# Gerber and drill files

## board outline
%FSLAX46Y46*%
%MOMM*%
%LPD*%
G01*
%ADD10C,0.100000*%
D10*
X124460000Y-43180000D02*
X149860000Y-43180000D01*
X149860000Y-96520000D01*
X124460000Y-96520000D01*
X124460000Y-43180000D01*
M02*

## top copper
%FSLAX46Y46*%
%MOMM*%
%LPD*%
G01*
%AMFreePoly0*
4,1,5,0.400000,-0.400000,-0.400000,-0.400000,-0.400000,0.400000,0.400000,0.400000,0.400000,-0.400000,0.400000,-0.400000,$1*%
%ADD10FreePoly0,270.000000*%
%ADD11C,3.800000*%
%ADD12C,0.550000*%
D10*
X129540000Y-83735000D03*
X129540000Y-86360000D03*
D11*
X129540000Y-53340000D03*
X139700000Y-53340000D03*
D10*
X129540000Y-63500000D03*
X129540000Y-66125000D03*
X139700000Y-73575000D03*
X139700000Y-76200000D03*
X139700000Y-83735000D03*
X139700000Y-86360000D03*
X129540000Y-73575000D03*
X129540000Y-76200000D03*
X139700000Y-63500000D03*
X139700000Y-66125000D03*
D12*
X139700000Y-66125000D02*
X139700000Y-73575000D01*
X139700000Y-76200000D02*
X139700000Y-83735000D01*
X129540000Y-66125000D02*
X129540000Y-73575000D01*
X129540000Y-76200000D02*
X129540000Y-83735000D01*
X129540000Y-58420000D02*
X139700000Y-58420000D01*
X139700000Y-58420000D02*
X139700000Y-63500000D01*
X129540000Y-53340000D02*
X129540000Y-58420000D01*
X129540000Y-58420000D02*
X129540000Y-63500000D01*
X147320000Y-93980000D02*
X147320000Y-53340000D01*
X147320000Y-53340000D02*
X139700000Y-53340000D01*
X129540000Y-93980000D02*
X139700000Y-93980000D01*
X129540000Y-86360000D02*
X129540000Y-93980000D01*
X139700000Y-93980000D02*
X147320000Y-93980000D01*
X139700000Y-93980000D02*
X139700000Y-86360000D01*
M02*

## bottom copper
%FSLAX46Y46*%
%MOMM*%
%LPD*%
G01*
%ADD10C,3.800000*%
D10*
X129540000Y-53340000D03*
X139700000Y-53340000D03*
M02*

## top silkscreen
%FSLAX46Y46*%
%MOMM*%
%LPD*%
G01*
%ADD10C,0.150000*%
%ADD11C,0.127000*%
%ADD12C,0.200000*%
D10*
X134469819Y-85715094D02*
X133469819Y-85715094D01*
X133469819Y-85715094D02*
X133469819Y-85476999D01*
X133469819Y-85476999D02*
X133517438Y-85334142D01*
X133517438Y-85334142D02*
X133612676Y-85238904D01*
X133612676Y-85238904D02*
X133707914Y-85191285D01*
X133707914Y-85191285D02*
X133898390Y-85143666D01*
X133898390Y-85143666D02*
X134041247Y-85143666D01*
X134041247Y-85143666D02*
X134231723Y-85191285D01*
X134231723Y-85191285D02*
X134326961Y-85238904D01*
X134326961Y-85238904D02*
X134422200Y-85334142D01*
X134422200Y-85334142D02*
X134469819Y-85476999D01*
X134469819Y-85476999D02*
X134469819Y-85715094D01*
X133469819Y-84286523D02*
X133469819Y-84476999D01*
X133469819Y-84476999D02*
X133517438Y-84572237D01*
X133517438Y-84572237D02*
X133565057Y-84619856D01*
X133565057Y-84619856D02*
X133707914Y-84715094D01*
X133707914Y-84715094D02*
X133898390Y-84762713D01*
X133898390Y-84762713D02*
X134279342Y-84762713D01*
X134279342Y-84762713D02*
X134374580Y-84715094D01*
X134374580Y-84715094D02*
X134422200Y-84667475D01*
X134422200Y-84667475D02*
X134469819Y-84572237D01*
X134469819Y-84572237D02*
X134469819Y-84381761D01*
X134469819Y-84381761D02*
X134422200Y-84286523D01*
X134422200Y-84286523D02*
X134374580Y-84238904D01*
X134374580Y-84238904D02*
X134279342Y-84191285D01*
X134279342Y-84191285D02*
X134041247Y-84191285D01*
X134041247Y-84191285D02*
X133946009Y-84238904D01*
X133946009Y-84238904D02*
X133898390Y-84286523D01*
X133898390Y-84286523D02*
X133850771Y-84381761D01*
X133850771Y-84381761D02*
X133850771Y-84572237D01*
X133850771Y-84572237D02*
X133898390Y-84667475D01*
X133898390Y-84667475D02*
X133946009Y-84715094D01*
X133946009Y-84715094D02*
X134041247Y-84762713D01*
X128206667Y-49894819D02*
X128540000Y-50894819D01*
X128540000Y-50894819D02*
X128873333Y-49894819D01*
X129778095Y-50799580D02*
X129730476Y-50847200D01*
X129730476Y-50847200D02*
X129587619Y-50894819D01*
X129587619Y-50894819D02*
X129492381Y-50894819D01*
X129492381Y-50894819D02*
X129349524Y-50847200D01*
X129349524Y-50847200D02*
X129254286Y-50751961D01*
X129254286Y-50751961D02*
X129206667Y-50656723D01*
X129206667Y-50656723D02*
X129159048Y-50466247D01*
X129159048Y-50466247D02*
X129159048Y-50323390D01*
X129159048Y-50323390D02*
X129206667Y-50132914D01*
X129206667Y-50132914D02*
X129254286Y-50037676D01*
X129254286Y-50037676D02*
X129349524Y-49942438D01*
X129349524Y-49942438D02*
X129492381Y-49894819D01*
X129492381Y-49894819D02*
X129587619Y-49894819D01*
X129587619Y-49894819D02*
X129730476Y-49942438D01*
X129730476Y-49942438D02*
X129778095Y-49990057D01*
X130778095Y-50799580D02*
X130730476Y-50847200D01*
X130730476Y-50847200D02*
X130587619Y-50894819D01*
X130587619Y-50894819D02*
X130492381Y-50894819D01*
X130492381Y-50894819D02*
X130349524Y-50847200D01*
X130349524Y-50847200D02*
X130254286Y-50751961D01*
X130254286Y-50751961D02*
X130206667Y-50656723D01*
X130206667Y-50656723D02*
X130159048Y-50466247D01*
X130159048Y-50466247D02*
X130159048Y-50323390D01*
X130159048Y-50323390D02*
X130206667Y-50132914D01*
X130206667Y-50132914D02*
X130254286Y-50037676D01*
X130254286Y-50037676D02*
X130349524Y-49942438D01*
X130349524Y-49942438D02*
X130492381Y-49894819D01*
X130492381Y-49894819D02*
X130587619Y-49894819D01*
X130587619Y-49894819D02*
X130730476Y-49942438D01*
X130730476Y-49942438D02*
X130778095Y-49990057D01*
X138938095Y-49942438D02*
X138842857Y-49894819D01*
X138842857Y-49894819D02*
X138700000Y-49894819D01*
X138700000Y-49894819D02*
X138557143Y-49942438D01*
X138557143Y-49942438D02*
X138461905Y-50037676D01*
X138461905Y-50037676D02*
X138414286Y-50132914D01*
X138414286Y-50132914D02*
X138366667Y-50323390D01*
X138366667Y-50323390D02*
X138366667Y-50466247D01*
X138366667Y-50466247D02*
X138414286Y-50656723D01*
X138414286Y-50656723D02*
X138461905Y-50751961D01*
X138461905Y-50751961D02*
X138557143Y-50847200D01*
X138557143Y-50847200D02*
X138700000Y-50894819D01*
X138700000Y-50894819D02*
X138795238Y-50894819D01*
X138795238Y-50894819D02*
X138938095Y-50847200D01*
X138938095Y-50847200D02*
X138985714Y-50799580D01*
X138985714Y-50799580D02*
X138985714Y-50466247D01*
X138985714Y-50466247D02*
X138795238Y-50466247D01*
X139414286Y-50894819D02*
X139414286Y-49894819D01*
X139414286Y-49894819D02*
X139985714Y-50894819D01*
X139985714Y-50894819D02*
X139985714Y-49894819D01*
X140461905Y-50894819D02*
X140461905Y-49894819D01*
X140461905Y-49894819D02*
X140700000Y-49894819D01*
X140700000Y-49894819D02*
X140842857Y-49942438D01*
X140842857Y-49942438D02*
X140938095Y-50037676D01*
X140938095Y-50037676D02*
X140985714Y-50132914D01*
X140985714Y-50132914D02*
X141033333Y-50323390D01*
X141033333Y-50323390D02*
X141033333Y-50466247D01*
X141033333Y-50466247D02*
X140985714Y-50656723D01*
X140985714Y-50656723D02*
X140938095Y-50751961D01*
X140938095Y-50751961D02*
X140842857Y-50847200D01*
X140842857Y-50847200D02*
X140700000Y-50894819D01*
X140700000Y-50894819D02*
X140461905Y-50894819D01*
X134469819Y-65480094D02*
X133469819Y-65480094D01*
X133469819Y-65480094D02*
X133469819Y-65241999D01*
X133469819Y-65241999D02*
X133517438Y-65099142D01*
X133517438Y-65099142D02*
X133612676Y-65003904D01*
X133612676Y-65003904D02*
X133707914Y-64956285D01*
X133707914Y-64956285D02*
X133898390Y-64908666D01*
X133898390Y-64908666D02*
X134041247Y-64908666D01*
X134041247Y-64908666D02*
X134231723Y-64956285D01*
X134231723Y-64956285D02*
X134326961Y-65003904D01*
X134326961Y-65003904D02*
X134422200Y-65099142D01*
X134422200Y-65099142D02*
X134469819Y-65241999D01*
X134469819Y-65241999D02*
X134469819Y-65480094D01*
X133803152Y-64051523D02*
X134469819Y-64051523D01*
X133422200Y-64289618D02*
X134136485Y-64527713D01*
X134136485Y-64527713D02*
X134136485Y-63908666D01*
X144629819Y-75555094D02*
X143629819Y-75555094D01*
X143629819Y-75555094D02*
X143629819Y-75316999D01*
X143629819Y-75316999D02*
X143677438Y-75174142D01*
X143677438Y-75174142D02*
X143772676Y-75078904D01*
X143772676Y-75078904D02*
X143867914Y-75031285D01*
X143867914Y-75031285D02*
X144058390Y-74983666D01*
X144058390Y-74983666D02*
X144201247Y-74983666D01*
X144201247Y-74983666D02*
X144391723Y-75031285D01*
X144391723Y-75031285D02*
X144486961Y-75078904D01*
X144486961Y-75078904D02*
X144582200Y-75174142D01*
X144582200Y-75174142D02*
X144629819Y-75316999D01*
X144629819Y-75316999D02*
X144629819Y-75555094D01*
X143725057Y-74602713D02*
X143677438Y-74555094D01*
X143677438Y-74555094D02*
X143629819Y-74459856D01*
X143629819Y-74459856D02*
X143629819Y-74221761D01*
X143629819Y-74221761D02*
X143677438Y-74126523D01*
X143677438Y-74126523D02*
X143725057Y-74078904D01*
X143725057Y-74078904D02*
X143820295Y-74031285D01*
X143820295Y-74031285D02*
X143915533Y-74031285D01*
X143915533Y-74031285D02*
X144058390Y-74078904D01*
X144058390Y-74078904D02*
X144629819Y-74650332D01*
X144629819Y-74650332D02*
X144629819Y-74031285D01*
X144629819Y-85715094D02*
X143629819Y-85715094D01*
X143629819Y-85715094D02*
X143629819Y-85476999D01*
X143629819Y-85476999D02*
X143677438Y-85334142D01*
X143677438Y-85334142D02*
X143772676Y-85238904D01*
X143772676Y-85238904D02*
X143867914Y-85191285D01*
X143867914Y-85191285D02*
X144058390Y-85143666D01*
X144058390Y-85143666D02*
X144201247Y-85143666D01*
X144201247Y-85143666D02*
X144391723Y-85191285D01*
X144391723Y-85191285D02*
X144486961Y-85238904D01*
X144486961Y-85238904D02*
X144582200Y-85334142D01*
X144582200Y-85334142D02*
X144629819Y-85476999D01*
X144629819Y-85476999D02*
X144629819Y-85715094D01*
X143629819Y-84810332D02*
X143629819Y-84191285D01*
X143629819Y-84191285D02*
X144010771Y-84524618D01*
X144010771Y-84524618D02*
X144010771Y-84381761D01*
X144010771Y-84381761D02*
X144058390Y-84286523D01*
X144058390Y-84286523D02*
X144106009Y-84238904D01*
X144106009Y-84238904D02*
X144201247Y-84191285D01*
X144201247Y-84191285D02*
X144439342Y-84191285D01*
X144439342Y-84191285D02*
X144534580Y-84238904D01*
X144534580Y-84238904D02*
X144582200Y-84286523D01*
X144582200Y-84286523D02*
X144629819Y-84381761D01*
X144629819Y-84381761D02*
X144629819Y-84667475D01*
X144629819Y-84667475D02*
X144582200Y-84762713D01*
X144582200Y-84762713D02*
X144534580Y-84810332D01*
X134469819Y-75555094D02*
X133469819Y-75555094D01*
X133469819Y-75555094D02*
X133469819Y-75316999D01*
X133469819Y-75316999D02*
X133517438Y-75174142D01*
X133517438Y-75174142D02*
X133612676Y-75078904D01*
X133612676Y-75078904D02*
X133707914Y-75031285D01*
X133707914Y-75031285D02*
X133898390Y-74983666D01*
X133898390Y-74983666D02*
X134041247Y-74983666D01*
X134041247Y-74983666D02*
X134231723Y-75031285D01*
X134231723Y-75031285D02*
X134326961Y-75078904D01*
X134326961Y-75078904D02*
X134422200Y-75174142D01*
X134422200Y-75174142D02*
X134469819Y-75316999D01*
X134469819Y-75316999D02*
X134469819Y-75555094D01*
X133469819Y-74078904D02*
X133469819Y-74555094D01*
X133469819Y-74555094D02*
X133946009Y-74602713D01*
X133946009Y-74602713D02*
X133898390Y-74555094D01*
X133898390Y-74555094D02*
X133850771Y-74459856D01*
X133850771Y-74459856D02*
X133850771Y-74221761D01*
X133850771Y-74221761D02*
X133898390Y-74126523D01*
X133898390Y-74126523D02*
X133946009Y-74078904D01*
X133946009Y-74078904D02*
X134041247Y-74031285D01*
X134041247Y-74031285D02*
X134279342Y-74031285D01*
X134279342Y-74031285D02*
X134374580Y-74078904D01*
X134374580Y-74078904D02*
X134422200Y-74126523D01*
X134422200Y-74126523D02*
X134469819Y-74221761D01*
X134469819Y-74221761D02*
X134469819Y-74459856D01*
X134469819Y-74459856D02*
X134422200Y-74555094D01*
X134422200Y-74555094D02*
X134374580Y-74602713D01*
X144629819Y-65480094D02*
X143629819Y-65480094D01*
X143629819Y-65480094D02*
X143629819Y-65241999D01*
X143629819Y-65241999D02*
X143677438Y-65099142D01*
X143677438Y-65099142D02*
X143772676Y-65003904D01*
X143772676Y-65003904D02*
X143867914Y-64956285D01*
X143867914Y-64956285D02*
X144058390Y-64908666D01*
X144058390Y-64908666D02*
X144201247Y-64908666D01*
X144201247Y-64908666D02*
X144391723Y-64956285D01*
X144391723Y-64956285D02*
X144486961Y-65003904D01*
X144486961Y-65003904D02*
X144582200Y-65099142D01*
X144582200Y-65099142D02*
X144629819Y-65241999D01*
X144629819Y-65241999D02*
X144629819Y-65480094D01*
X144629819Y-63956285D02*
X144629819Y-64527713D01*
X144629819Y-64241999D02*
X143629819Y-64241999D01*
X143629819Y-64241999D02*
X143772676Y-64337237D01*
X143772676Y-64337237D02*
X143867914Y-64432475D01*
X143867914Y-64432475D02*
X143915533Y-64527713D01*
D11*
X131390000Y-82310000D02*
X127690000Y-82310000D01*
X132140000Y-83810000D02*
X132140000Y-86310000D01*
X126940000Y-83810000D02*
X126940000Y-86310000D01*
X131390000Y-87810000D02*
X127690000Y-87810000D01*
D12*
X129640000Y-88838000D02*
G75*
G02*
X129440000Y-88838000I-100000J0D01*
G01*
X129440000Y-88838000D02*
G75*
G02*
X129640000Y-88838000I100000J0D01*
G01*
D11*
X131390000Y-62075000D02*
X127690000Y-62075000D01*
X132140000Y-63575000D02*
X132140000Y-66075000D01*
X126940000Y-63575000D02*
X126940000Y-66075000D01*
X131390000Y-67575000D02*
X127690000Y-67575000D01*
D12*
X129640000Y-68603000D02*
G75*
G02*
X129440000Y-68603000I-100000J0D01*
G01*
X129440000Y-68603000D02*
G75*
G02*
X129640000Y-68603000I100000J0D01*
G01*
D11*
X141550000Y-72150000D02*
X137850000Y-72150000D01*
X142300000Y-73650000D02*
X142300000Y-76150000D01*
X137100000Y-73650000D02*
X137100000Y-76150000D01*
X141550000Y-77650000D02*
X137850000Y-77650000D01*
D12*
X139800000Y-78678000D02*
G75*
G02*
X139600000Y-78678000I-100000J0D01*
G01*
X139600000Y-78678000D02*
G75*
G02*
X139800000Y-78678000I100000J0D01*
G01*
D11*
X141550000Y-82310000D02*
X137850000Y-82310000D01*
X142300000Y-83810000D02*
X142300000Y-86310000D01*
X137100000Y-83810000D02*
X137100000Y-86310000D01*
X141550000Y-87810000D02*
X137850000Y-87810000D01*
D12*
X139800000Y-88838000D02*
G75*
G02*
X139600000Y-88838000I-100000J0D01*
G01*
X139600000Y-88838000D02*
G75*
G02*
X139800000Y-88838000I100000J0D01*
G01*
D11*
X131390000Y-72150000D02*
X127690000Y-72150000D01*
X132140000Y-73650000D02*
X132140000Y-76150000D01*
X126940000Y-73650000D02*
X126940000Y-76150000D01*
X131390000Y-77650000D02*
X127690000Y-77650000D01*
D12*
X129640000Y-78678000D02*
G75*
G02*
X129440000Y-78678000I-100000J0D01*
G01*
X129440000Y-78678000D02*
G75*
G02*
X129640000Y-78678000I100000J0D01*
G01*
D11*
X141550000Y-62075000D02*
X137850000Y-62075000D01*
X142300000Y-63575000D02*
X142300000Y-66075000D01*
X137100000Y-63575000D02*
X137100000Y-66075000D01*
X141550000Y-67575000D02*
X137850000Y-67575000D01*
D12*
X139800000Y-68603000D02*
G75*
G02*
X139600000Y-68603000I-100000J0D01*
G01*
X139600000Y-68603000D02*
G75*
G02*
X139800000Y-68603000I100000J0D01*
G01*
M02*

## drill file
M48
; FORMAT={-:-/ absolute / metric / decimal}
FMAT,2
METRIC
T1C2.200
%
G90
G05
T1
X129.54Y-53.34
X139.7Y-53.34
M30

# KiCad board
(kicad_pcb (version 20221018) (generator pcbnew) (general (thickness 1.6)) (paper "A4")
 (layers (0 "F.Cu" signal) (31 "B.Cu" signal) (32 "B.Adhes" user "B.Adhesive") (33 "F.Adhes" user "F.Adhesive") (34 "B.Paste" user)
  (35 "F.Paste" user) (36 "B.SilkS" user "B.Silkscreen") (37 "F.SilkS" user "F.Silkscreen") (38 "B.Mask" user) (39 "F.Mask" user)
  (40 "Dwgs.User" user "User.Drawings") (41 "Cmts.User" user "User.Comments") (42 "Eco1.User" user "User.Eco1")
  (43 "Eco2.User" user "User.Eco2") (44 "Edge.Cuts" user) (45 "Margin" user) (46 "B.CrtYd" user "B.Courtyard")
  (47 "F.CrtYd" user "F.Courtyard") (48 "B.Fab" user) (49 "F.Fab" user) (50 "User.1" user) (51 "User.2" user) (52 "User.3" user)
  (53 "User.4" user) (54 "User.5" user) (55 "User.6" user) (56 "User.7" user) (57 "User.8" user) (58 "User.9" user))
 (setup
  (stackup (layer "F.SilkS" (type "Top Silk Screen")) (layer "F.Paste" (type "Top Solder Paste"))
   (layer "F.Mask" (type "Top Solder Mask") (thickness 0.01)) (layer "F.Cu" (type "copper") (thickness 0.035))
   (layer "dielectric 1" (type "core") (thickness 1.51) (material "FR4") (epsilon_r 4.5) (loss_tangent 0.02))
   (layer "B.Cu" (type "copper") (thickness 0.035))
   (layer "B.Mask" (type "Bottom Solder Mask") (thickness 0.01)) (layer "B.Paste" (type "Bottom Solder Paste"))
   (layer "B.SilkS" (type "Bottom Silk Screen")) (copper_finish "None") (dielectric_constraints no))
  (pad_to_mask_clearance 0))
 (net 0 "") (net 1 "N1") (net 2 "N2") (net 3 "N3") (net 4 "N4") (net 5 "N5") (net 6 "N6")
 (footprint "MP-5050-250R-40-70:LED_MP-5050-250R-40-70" (layer "F.Cu") (at 129.54 85.06 -90)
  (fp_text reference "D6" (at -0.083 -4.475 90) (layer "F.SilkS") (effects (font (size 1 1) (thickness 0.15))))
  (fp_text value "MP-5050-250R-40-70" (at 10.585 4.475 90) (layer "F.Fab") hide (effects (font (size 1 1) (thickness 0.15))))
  (fp_line (start -2.75 -1.85) (end -2.75 1.85) (stroke (width 0.127) (type solid)) (layer "F.SilkS"))
  (fp_line (start -1.25 -2.6) (end 1.25 -2.6) (stroke (width 0.127) (type solid)) (layer "F.SilkS"))
  (fp_line (start -1.25 2.6) (end 1.25 2.6) (stroke (width 0.127) (type solid)) (layer "F.SilkS"))
  (fp_line (start 2.75 -1.85) (end 2.75 1.85) (stroke (width 0.127) (type solid)) (layer "F.SilkS"))
  (fp_circle (center 3.778 0) (end 3.878 0) (stroke (width 0.2) (type solid)) (fill none) (layer "F.SilkS"))
  (pad "A" smd custom (at -1.325 0 270) (size 0.8 0.8) (layers "F.Cu") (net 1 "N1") (options (clearance outline) (anchor rect)) (primitives))
  (pad "C" smd custom (at 1.3 0 270) (size 0.8 0.8) (layers "F.Cu") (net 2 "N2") (options (clearance outline) (anchor rect)) (primitives)))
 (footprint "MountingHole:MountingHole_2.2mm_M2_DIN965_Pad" (layer "F.Cu") (at 129.54 53.34)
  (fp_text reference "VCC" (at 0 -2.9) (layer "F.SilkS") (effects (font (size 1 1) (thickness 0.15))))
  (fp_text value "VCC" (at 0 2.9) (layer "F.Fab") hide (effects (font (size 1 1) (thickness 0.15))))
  (pad "1" thru_hole circle (at 0 0) (size 3.8 3.8) (drill 2.2) (layers "*.Cu" "*.Mask") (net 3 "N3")))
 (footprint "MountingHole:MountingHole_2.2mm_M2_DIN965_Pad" (layer "F.Cu") (at 139.7 53.34)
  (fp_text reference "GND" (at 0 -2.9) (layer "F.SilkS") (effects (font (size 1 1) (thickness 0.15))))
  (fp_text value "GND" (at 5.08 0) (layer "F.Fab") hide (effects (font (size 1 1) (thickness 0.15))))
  (pad "1" thru_hole circle (at 0 0) (size 3.8 3.8) (drill 2.2) (layers "*.Cu" "*.Mask") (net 2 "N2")))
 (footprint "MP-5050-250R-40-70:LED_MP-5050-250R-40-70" (layer "F.Cu") (at 129.54 64.825 -90)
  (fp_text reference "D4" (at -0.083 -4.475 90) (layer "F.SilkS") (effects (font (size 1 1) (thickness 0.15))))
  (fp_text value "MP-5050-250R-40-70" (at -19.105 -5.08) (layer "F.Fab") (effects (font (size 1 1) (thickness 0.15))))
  (fp_line (start -2.75 -1.85) (end -2.75 1.85) (stroke (width 0.127) (type solid)) (layer "F.SilkS"))
  (fp_line (start -1.25 -2.6) (end 1.25 -2.6) (stroke (width 0.127) (type solid)) (layer "F.SilkS"))
  (fp_line (start -1.25 2.6) (end 1.25 2.6) (stroke (width 0.127) (type solid)) (layer "F.SilkS"))
  (fp_line (start 2.75 -1.85) (end 2.75 1.85) (stroke (width 0.127) (type solid)) (layer "F.SilkS"))
  (fp_circle (center 3.778 0) (end 3.878 0) (stroke (width 0.2) (type solid)) (fill none) (layer "F.SilkS"))
  (pad "A" smd custom (at -1.325 0 270) (size 0.8 0.8) (layers "F.Cu") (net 3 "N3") (options (clearance outline) (anchor rect)) (primitives))
  (pad "C" smd custom (at 1.3 0 270) (size 0.8 0.8) (layers "F.Cu") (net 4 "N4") (options (clearance outline) (anchor rect)) (primitives)))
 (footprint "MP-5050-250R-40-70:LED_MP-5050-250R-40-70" (layer "F.Cu") (at 139.7 74.9 -90)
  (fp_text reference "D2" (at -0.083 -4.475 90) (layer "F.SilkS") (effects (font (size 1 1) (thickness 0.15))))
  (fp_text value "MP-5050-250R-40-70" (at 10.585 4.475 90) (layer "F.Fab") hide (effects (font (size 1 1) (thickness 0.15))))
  (fp_line (start -2.75 -1.85) (end -2.75 1.85) (stroke (width 0.127) (type solid)) (layer "F.SilkS"))
  (fp_line (start -1.25 -2.6) (end 1.25 -2.6) (stroke (width 0.127) (type solid)) (layer "F.SilkS"))
  (fp_line (start -1.25 2.6) (end 1.25 2.6) (stroke (width 0.127) (type solid)) (layer "F.SilkS"))
  (fp_line (start 2.75 -1.85) (end 2.75 1.85) (stroke (width 0.127) (type solid)) (layer "F.SilkS"))
  (fp_circle (center 3.778 0) (end 3.878 0) (stroke (width 0.2) (type solid)) (fill none) (layer "F.SilkS"))
  (pad "A" smd custom (at -1.325 0 270) (size 0.8 0.8) (layers "F.Cu") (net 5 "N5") (options (clearance outline) (anchor rect)) (primitives))
  (pad "C" smd custom (at 1.3 0 270) (size 0.8 0.8) (layers "F.Cu") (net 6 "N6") (options (clearance outline) (anchor rect)) (primitives)))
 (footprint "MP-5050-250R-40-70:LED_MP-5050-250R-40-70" (layer "F.Cu") (at 139.7 85.06 -90)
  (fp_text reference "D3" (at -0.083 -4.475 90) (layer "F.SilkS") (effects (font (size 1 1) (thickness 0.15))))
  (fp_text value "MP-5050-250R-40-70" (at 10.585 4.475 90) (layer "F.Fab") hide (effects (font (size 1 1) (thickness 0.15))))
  (fp_line (start -2.75 -1.85) (end -2.75 1.85) (stroke (width 0.127) (type solid)) (layer "F.SilkS"))
  (fp_line (start -1.25 -2.6) (end 1.25 -2.6) (stroke (width 0.127) (type solid)) (layer "F.SilkS"))
  (fp_line (start -1.25 2.6) (end 1.25 2.6) (stroke (width 0.127) (type solid)) (layer "F.SilkS"))
  (fp_line (start 2.75 -1.85) (end 2.75 1.85) (stroke (width 0.127) (type solid)) (layer "F.SilkS"))
  (fp_circle (center 3.778 0) (end 3.878 0) (stroke (width 0.2) (type solid)) (fill none) (layer "F.SilkS"))
  (pad "A" smd custom (at -1.325 0 270) (size 0.8 0.8) (layers "F.Cu") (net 6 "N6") (options (clearance outline) (anchor rect)) (primitives))
  (pad "C" smd custom (at 1.3 0 270) (size 0.8 0.8) (layers "F.Cu") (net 2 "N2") (options (clearance outline) (anchor rect)) (primitives)))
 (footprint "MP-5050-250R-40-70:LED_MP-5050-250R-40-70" (layer "F.Cu") (at 129.54 74.9 -90)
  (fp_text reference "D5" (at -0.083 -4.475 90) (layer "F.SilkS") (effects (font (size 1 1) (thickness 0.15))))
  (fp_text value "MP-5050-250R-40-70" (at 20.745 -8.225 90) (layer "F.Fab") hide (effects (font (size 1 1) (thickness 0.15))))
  (fp_line (start -2.75 -1.85) (end -2.75 1.85) (stroke (width 0.127) (type solid)) (layer "F.SilkS"))
  (fp_line (start -1.25 -2.6) (end 1.25 -2.6) (stroke (width 0.127) (type solid)) (layer "F.SilkS"))
  (fp_line (start -1.25 2.6) (end 1.25 2.6) (stroke (width 0.127) (type solid)) (layer "F.SilkS"))
  (fp_line (start 2.75 -1.85) (end 2.75 1.85) (stroke (width 0.127) (type solid)) (layer "F.SilkS"))
  (fp_circle (center 3.778 0) (end 3.878 0) (stroke (width 0.2) (type solid)) (fill none) (layer "F.SilkS"))
  (pad "A" smd custom (at -1.325 0 270) (size 0.8 0.8) (layers "F.Cu") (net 4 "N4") (options (clearance outline) (anchor rect)) (primitives))
  (pad "C" smd custom (at 1.3 0 270) (size 0.8 0.8) (layers "F.Cu") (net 1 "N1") (options (clearance outline) (anchor rect)) (primitives)))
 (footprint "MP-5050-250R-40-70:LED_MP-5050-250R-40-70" (layer "F.Cu") (at 139.7 64.825 -90)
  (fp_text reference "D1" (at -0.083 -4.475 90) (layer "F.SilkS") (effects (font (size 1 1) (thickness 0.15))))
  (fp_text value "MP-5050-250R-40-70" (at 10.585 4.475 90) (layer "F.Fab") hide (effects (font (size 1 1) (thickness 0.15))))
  (fp_line (start -2.75 -1.85) (end -2.75 1.85) (stroke (width 0.127) (type solid)) (layer "F.SilkS"))
  (fp_line (start -1.25 -2.6) (end 1.25 -2.6) (stroke (width 0.127) (type solid)) (layer "F.SilkS"))
  (fp_line (start -1.25 2.6) (end 1.25 2.6) (stroke (width 0.127) (type solid)) (layer "F.SilkS"))
  (fp_line (start 2.75 -1.85) (end 2.75 1.85) (stroke (width 0.127) (type solid)) (layer "F.SilkS"))
  (fp_circle (center 3.778 0) (end 3.878 0) (stroke (width 0.2) (type solid)) (fill none) (layer "F.SilkS"))
  (pad "A" smd custom (at -1.325 0 270) (size 0.8 0.8) (layers "F.Cu") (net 3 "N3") (options (clearance outline) (anchor rect)) (primitives))
  (pad "C" smd custom (at 1.3 0 270) (size 0.8 0.8) (layers "F.Cu") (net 5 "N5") (options (clearance outline) (anchor rect)) (primitives)))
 (gr_rect (start 124.46 43.18) (end 149.86 96.52) (stroke (width 0.1) (type default)) (fill none) (layer "Edge.Cuts"))
 (segment (start 139.7 66.125) (end 139.7 73.575) (width 0.55) (layer "F.Cu") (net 5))
 (segment (start 139.7 76.2) (end 139.7 83.735) (width 0.55) (layer "F.Cu") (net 6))
 (segment (start 129.54 66.125) (end 129.54 73.575) (width 0.55) (layer "F.Cu") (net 4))
 (segment (start 129.54 76.2) (end 129.54 83.735) (width 0.55) (layer "F.Cu") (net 1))
 (segment (start 129.54 58.42) (end 139.7 58.42) (width 0.55) (layer "F.Cu") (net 3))
 (segment (start 139.7 58.42) (end 139.7 63.5) (width 0.55) (layer "F.Cu") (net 3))
 (segment (start 129.54 53.34) (end 129.54 58.42) (width 0.55) (layer "F.Cu") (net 3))
 (segment (start 129.54 58.42) (end 129.54 63.5) (width 0.55) (layer "F.Cu") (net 3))
 (segment (start 147.32 93.98) (end 147.32 53.34) (width 0.55) (layer "F.Cu") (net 2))
 (segment (start 147.32 53.34) (end 139.7 53.34) (width 0.55) (layer "F.Cu") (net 2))
 (segment (start 129.54 93.98) (end 139.7 93.98) (width 0.55) (layer "F.Cu") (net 2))
 (segment (start 129.54 86.36) (end 129.54 93.98) (width 0.55) (layer "F.Cu") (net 2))
 (segment (start 139.7 93.98) (end 147.32 93.98) (width 0.55) (layer "F.Cu") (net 2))
 (segment (start 139.7 93.98) (end 139.7 86.36) (width 0.55) (layer "F.Cu") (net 2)))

